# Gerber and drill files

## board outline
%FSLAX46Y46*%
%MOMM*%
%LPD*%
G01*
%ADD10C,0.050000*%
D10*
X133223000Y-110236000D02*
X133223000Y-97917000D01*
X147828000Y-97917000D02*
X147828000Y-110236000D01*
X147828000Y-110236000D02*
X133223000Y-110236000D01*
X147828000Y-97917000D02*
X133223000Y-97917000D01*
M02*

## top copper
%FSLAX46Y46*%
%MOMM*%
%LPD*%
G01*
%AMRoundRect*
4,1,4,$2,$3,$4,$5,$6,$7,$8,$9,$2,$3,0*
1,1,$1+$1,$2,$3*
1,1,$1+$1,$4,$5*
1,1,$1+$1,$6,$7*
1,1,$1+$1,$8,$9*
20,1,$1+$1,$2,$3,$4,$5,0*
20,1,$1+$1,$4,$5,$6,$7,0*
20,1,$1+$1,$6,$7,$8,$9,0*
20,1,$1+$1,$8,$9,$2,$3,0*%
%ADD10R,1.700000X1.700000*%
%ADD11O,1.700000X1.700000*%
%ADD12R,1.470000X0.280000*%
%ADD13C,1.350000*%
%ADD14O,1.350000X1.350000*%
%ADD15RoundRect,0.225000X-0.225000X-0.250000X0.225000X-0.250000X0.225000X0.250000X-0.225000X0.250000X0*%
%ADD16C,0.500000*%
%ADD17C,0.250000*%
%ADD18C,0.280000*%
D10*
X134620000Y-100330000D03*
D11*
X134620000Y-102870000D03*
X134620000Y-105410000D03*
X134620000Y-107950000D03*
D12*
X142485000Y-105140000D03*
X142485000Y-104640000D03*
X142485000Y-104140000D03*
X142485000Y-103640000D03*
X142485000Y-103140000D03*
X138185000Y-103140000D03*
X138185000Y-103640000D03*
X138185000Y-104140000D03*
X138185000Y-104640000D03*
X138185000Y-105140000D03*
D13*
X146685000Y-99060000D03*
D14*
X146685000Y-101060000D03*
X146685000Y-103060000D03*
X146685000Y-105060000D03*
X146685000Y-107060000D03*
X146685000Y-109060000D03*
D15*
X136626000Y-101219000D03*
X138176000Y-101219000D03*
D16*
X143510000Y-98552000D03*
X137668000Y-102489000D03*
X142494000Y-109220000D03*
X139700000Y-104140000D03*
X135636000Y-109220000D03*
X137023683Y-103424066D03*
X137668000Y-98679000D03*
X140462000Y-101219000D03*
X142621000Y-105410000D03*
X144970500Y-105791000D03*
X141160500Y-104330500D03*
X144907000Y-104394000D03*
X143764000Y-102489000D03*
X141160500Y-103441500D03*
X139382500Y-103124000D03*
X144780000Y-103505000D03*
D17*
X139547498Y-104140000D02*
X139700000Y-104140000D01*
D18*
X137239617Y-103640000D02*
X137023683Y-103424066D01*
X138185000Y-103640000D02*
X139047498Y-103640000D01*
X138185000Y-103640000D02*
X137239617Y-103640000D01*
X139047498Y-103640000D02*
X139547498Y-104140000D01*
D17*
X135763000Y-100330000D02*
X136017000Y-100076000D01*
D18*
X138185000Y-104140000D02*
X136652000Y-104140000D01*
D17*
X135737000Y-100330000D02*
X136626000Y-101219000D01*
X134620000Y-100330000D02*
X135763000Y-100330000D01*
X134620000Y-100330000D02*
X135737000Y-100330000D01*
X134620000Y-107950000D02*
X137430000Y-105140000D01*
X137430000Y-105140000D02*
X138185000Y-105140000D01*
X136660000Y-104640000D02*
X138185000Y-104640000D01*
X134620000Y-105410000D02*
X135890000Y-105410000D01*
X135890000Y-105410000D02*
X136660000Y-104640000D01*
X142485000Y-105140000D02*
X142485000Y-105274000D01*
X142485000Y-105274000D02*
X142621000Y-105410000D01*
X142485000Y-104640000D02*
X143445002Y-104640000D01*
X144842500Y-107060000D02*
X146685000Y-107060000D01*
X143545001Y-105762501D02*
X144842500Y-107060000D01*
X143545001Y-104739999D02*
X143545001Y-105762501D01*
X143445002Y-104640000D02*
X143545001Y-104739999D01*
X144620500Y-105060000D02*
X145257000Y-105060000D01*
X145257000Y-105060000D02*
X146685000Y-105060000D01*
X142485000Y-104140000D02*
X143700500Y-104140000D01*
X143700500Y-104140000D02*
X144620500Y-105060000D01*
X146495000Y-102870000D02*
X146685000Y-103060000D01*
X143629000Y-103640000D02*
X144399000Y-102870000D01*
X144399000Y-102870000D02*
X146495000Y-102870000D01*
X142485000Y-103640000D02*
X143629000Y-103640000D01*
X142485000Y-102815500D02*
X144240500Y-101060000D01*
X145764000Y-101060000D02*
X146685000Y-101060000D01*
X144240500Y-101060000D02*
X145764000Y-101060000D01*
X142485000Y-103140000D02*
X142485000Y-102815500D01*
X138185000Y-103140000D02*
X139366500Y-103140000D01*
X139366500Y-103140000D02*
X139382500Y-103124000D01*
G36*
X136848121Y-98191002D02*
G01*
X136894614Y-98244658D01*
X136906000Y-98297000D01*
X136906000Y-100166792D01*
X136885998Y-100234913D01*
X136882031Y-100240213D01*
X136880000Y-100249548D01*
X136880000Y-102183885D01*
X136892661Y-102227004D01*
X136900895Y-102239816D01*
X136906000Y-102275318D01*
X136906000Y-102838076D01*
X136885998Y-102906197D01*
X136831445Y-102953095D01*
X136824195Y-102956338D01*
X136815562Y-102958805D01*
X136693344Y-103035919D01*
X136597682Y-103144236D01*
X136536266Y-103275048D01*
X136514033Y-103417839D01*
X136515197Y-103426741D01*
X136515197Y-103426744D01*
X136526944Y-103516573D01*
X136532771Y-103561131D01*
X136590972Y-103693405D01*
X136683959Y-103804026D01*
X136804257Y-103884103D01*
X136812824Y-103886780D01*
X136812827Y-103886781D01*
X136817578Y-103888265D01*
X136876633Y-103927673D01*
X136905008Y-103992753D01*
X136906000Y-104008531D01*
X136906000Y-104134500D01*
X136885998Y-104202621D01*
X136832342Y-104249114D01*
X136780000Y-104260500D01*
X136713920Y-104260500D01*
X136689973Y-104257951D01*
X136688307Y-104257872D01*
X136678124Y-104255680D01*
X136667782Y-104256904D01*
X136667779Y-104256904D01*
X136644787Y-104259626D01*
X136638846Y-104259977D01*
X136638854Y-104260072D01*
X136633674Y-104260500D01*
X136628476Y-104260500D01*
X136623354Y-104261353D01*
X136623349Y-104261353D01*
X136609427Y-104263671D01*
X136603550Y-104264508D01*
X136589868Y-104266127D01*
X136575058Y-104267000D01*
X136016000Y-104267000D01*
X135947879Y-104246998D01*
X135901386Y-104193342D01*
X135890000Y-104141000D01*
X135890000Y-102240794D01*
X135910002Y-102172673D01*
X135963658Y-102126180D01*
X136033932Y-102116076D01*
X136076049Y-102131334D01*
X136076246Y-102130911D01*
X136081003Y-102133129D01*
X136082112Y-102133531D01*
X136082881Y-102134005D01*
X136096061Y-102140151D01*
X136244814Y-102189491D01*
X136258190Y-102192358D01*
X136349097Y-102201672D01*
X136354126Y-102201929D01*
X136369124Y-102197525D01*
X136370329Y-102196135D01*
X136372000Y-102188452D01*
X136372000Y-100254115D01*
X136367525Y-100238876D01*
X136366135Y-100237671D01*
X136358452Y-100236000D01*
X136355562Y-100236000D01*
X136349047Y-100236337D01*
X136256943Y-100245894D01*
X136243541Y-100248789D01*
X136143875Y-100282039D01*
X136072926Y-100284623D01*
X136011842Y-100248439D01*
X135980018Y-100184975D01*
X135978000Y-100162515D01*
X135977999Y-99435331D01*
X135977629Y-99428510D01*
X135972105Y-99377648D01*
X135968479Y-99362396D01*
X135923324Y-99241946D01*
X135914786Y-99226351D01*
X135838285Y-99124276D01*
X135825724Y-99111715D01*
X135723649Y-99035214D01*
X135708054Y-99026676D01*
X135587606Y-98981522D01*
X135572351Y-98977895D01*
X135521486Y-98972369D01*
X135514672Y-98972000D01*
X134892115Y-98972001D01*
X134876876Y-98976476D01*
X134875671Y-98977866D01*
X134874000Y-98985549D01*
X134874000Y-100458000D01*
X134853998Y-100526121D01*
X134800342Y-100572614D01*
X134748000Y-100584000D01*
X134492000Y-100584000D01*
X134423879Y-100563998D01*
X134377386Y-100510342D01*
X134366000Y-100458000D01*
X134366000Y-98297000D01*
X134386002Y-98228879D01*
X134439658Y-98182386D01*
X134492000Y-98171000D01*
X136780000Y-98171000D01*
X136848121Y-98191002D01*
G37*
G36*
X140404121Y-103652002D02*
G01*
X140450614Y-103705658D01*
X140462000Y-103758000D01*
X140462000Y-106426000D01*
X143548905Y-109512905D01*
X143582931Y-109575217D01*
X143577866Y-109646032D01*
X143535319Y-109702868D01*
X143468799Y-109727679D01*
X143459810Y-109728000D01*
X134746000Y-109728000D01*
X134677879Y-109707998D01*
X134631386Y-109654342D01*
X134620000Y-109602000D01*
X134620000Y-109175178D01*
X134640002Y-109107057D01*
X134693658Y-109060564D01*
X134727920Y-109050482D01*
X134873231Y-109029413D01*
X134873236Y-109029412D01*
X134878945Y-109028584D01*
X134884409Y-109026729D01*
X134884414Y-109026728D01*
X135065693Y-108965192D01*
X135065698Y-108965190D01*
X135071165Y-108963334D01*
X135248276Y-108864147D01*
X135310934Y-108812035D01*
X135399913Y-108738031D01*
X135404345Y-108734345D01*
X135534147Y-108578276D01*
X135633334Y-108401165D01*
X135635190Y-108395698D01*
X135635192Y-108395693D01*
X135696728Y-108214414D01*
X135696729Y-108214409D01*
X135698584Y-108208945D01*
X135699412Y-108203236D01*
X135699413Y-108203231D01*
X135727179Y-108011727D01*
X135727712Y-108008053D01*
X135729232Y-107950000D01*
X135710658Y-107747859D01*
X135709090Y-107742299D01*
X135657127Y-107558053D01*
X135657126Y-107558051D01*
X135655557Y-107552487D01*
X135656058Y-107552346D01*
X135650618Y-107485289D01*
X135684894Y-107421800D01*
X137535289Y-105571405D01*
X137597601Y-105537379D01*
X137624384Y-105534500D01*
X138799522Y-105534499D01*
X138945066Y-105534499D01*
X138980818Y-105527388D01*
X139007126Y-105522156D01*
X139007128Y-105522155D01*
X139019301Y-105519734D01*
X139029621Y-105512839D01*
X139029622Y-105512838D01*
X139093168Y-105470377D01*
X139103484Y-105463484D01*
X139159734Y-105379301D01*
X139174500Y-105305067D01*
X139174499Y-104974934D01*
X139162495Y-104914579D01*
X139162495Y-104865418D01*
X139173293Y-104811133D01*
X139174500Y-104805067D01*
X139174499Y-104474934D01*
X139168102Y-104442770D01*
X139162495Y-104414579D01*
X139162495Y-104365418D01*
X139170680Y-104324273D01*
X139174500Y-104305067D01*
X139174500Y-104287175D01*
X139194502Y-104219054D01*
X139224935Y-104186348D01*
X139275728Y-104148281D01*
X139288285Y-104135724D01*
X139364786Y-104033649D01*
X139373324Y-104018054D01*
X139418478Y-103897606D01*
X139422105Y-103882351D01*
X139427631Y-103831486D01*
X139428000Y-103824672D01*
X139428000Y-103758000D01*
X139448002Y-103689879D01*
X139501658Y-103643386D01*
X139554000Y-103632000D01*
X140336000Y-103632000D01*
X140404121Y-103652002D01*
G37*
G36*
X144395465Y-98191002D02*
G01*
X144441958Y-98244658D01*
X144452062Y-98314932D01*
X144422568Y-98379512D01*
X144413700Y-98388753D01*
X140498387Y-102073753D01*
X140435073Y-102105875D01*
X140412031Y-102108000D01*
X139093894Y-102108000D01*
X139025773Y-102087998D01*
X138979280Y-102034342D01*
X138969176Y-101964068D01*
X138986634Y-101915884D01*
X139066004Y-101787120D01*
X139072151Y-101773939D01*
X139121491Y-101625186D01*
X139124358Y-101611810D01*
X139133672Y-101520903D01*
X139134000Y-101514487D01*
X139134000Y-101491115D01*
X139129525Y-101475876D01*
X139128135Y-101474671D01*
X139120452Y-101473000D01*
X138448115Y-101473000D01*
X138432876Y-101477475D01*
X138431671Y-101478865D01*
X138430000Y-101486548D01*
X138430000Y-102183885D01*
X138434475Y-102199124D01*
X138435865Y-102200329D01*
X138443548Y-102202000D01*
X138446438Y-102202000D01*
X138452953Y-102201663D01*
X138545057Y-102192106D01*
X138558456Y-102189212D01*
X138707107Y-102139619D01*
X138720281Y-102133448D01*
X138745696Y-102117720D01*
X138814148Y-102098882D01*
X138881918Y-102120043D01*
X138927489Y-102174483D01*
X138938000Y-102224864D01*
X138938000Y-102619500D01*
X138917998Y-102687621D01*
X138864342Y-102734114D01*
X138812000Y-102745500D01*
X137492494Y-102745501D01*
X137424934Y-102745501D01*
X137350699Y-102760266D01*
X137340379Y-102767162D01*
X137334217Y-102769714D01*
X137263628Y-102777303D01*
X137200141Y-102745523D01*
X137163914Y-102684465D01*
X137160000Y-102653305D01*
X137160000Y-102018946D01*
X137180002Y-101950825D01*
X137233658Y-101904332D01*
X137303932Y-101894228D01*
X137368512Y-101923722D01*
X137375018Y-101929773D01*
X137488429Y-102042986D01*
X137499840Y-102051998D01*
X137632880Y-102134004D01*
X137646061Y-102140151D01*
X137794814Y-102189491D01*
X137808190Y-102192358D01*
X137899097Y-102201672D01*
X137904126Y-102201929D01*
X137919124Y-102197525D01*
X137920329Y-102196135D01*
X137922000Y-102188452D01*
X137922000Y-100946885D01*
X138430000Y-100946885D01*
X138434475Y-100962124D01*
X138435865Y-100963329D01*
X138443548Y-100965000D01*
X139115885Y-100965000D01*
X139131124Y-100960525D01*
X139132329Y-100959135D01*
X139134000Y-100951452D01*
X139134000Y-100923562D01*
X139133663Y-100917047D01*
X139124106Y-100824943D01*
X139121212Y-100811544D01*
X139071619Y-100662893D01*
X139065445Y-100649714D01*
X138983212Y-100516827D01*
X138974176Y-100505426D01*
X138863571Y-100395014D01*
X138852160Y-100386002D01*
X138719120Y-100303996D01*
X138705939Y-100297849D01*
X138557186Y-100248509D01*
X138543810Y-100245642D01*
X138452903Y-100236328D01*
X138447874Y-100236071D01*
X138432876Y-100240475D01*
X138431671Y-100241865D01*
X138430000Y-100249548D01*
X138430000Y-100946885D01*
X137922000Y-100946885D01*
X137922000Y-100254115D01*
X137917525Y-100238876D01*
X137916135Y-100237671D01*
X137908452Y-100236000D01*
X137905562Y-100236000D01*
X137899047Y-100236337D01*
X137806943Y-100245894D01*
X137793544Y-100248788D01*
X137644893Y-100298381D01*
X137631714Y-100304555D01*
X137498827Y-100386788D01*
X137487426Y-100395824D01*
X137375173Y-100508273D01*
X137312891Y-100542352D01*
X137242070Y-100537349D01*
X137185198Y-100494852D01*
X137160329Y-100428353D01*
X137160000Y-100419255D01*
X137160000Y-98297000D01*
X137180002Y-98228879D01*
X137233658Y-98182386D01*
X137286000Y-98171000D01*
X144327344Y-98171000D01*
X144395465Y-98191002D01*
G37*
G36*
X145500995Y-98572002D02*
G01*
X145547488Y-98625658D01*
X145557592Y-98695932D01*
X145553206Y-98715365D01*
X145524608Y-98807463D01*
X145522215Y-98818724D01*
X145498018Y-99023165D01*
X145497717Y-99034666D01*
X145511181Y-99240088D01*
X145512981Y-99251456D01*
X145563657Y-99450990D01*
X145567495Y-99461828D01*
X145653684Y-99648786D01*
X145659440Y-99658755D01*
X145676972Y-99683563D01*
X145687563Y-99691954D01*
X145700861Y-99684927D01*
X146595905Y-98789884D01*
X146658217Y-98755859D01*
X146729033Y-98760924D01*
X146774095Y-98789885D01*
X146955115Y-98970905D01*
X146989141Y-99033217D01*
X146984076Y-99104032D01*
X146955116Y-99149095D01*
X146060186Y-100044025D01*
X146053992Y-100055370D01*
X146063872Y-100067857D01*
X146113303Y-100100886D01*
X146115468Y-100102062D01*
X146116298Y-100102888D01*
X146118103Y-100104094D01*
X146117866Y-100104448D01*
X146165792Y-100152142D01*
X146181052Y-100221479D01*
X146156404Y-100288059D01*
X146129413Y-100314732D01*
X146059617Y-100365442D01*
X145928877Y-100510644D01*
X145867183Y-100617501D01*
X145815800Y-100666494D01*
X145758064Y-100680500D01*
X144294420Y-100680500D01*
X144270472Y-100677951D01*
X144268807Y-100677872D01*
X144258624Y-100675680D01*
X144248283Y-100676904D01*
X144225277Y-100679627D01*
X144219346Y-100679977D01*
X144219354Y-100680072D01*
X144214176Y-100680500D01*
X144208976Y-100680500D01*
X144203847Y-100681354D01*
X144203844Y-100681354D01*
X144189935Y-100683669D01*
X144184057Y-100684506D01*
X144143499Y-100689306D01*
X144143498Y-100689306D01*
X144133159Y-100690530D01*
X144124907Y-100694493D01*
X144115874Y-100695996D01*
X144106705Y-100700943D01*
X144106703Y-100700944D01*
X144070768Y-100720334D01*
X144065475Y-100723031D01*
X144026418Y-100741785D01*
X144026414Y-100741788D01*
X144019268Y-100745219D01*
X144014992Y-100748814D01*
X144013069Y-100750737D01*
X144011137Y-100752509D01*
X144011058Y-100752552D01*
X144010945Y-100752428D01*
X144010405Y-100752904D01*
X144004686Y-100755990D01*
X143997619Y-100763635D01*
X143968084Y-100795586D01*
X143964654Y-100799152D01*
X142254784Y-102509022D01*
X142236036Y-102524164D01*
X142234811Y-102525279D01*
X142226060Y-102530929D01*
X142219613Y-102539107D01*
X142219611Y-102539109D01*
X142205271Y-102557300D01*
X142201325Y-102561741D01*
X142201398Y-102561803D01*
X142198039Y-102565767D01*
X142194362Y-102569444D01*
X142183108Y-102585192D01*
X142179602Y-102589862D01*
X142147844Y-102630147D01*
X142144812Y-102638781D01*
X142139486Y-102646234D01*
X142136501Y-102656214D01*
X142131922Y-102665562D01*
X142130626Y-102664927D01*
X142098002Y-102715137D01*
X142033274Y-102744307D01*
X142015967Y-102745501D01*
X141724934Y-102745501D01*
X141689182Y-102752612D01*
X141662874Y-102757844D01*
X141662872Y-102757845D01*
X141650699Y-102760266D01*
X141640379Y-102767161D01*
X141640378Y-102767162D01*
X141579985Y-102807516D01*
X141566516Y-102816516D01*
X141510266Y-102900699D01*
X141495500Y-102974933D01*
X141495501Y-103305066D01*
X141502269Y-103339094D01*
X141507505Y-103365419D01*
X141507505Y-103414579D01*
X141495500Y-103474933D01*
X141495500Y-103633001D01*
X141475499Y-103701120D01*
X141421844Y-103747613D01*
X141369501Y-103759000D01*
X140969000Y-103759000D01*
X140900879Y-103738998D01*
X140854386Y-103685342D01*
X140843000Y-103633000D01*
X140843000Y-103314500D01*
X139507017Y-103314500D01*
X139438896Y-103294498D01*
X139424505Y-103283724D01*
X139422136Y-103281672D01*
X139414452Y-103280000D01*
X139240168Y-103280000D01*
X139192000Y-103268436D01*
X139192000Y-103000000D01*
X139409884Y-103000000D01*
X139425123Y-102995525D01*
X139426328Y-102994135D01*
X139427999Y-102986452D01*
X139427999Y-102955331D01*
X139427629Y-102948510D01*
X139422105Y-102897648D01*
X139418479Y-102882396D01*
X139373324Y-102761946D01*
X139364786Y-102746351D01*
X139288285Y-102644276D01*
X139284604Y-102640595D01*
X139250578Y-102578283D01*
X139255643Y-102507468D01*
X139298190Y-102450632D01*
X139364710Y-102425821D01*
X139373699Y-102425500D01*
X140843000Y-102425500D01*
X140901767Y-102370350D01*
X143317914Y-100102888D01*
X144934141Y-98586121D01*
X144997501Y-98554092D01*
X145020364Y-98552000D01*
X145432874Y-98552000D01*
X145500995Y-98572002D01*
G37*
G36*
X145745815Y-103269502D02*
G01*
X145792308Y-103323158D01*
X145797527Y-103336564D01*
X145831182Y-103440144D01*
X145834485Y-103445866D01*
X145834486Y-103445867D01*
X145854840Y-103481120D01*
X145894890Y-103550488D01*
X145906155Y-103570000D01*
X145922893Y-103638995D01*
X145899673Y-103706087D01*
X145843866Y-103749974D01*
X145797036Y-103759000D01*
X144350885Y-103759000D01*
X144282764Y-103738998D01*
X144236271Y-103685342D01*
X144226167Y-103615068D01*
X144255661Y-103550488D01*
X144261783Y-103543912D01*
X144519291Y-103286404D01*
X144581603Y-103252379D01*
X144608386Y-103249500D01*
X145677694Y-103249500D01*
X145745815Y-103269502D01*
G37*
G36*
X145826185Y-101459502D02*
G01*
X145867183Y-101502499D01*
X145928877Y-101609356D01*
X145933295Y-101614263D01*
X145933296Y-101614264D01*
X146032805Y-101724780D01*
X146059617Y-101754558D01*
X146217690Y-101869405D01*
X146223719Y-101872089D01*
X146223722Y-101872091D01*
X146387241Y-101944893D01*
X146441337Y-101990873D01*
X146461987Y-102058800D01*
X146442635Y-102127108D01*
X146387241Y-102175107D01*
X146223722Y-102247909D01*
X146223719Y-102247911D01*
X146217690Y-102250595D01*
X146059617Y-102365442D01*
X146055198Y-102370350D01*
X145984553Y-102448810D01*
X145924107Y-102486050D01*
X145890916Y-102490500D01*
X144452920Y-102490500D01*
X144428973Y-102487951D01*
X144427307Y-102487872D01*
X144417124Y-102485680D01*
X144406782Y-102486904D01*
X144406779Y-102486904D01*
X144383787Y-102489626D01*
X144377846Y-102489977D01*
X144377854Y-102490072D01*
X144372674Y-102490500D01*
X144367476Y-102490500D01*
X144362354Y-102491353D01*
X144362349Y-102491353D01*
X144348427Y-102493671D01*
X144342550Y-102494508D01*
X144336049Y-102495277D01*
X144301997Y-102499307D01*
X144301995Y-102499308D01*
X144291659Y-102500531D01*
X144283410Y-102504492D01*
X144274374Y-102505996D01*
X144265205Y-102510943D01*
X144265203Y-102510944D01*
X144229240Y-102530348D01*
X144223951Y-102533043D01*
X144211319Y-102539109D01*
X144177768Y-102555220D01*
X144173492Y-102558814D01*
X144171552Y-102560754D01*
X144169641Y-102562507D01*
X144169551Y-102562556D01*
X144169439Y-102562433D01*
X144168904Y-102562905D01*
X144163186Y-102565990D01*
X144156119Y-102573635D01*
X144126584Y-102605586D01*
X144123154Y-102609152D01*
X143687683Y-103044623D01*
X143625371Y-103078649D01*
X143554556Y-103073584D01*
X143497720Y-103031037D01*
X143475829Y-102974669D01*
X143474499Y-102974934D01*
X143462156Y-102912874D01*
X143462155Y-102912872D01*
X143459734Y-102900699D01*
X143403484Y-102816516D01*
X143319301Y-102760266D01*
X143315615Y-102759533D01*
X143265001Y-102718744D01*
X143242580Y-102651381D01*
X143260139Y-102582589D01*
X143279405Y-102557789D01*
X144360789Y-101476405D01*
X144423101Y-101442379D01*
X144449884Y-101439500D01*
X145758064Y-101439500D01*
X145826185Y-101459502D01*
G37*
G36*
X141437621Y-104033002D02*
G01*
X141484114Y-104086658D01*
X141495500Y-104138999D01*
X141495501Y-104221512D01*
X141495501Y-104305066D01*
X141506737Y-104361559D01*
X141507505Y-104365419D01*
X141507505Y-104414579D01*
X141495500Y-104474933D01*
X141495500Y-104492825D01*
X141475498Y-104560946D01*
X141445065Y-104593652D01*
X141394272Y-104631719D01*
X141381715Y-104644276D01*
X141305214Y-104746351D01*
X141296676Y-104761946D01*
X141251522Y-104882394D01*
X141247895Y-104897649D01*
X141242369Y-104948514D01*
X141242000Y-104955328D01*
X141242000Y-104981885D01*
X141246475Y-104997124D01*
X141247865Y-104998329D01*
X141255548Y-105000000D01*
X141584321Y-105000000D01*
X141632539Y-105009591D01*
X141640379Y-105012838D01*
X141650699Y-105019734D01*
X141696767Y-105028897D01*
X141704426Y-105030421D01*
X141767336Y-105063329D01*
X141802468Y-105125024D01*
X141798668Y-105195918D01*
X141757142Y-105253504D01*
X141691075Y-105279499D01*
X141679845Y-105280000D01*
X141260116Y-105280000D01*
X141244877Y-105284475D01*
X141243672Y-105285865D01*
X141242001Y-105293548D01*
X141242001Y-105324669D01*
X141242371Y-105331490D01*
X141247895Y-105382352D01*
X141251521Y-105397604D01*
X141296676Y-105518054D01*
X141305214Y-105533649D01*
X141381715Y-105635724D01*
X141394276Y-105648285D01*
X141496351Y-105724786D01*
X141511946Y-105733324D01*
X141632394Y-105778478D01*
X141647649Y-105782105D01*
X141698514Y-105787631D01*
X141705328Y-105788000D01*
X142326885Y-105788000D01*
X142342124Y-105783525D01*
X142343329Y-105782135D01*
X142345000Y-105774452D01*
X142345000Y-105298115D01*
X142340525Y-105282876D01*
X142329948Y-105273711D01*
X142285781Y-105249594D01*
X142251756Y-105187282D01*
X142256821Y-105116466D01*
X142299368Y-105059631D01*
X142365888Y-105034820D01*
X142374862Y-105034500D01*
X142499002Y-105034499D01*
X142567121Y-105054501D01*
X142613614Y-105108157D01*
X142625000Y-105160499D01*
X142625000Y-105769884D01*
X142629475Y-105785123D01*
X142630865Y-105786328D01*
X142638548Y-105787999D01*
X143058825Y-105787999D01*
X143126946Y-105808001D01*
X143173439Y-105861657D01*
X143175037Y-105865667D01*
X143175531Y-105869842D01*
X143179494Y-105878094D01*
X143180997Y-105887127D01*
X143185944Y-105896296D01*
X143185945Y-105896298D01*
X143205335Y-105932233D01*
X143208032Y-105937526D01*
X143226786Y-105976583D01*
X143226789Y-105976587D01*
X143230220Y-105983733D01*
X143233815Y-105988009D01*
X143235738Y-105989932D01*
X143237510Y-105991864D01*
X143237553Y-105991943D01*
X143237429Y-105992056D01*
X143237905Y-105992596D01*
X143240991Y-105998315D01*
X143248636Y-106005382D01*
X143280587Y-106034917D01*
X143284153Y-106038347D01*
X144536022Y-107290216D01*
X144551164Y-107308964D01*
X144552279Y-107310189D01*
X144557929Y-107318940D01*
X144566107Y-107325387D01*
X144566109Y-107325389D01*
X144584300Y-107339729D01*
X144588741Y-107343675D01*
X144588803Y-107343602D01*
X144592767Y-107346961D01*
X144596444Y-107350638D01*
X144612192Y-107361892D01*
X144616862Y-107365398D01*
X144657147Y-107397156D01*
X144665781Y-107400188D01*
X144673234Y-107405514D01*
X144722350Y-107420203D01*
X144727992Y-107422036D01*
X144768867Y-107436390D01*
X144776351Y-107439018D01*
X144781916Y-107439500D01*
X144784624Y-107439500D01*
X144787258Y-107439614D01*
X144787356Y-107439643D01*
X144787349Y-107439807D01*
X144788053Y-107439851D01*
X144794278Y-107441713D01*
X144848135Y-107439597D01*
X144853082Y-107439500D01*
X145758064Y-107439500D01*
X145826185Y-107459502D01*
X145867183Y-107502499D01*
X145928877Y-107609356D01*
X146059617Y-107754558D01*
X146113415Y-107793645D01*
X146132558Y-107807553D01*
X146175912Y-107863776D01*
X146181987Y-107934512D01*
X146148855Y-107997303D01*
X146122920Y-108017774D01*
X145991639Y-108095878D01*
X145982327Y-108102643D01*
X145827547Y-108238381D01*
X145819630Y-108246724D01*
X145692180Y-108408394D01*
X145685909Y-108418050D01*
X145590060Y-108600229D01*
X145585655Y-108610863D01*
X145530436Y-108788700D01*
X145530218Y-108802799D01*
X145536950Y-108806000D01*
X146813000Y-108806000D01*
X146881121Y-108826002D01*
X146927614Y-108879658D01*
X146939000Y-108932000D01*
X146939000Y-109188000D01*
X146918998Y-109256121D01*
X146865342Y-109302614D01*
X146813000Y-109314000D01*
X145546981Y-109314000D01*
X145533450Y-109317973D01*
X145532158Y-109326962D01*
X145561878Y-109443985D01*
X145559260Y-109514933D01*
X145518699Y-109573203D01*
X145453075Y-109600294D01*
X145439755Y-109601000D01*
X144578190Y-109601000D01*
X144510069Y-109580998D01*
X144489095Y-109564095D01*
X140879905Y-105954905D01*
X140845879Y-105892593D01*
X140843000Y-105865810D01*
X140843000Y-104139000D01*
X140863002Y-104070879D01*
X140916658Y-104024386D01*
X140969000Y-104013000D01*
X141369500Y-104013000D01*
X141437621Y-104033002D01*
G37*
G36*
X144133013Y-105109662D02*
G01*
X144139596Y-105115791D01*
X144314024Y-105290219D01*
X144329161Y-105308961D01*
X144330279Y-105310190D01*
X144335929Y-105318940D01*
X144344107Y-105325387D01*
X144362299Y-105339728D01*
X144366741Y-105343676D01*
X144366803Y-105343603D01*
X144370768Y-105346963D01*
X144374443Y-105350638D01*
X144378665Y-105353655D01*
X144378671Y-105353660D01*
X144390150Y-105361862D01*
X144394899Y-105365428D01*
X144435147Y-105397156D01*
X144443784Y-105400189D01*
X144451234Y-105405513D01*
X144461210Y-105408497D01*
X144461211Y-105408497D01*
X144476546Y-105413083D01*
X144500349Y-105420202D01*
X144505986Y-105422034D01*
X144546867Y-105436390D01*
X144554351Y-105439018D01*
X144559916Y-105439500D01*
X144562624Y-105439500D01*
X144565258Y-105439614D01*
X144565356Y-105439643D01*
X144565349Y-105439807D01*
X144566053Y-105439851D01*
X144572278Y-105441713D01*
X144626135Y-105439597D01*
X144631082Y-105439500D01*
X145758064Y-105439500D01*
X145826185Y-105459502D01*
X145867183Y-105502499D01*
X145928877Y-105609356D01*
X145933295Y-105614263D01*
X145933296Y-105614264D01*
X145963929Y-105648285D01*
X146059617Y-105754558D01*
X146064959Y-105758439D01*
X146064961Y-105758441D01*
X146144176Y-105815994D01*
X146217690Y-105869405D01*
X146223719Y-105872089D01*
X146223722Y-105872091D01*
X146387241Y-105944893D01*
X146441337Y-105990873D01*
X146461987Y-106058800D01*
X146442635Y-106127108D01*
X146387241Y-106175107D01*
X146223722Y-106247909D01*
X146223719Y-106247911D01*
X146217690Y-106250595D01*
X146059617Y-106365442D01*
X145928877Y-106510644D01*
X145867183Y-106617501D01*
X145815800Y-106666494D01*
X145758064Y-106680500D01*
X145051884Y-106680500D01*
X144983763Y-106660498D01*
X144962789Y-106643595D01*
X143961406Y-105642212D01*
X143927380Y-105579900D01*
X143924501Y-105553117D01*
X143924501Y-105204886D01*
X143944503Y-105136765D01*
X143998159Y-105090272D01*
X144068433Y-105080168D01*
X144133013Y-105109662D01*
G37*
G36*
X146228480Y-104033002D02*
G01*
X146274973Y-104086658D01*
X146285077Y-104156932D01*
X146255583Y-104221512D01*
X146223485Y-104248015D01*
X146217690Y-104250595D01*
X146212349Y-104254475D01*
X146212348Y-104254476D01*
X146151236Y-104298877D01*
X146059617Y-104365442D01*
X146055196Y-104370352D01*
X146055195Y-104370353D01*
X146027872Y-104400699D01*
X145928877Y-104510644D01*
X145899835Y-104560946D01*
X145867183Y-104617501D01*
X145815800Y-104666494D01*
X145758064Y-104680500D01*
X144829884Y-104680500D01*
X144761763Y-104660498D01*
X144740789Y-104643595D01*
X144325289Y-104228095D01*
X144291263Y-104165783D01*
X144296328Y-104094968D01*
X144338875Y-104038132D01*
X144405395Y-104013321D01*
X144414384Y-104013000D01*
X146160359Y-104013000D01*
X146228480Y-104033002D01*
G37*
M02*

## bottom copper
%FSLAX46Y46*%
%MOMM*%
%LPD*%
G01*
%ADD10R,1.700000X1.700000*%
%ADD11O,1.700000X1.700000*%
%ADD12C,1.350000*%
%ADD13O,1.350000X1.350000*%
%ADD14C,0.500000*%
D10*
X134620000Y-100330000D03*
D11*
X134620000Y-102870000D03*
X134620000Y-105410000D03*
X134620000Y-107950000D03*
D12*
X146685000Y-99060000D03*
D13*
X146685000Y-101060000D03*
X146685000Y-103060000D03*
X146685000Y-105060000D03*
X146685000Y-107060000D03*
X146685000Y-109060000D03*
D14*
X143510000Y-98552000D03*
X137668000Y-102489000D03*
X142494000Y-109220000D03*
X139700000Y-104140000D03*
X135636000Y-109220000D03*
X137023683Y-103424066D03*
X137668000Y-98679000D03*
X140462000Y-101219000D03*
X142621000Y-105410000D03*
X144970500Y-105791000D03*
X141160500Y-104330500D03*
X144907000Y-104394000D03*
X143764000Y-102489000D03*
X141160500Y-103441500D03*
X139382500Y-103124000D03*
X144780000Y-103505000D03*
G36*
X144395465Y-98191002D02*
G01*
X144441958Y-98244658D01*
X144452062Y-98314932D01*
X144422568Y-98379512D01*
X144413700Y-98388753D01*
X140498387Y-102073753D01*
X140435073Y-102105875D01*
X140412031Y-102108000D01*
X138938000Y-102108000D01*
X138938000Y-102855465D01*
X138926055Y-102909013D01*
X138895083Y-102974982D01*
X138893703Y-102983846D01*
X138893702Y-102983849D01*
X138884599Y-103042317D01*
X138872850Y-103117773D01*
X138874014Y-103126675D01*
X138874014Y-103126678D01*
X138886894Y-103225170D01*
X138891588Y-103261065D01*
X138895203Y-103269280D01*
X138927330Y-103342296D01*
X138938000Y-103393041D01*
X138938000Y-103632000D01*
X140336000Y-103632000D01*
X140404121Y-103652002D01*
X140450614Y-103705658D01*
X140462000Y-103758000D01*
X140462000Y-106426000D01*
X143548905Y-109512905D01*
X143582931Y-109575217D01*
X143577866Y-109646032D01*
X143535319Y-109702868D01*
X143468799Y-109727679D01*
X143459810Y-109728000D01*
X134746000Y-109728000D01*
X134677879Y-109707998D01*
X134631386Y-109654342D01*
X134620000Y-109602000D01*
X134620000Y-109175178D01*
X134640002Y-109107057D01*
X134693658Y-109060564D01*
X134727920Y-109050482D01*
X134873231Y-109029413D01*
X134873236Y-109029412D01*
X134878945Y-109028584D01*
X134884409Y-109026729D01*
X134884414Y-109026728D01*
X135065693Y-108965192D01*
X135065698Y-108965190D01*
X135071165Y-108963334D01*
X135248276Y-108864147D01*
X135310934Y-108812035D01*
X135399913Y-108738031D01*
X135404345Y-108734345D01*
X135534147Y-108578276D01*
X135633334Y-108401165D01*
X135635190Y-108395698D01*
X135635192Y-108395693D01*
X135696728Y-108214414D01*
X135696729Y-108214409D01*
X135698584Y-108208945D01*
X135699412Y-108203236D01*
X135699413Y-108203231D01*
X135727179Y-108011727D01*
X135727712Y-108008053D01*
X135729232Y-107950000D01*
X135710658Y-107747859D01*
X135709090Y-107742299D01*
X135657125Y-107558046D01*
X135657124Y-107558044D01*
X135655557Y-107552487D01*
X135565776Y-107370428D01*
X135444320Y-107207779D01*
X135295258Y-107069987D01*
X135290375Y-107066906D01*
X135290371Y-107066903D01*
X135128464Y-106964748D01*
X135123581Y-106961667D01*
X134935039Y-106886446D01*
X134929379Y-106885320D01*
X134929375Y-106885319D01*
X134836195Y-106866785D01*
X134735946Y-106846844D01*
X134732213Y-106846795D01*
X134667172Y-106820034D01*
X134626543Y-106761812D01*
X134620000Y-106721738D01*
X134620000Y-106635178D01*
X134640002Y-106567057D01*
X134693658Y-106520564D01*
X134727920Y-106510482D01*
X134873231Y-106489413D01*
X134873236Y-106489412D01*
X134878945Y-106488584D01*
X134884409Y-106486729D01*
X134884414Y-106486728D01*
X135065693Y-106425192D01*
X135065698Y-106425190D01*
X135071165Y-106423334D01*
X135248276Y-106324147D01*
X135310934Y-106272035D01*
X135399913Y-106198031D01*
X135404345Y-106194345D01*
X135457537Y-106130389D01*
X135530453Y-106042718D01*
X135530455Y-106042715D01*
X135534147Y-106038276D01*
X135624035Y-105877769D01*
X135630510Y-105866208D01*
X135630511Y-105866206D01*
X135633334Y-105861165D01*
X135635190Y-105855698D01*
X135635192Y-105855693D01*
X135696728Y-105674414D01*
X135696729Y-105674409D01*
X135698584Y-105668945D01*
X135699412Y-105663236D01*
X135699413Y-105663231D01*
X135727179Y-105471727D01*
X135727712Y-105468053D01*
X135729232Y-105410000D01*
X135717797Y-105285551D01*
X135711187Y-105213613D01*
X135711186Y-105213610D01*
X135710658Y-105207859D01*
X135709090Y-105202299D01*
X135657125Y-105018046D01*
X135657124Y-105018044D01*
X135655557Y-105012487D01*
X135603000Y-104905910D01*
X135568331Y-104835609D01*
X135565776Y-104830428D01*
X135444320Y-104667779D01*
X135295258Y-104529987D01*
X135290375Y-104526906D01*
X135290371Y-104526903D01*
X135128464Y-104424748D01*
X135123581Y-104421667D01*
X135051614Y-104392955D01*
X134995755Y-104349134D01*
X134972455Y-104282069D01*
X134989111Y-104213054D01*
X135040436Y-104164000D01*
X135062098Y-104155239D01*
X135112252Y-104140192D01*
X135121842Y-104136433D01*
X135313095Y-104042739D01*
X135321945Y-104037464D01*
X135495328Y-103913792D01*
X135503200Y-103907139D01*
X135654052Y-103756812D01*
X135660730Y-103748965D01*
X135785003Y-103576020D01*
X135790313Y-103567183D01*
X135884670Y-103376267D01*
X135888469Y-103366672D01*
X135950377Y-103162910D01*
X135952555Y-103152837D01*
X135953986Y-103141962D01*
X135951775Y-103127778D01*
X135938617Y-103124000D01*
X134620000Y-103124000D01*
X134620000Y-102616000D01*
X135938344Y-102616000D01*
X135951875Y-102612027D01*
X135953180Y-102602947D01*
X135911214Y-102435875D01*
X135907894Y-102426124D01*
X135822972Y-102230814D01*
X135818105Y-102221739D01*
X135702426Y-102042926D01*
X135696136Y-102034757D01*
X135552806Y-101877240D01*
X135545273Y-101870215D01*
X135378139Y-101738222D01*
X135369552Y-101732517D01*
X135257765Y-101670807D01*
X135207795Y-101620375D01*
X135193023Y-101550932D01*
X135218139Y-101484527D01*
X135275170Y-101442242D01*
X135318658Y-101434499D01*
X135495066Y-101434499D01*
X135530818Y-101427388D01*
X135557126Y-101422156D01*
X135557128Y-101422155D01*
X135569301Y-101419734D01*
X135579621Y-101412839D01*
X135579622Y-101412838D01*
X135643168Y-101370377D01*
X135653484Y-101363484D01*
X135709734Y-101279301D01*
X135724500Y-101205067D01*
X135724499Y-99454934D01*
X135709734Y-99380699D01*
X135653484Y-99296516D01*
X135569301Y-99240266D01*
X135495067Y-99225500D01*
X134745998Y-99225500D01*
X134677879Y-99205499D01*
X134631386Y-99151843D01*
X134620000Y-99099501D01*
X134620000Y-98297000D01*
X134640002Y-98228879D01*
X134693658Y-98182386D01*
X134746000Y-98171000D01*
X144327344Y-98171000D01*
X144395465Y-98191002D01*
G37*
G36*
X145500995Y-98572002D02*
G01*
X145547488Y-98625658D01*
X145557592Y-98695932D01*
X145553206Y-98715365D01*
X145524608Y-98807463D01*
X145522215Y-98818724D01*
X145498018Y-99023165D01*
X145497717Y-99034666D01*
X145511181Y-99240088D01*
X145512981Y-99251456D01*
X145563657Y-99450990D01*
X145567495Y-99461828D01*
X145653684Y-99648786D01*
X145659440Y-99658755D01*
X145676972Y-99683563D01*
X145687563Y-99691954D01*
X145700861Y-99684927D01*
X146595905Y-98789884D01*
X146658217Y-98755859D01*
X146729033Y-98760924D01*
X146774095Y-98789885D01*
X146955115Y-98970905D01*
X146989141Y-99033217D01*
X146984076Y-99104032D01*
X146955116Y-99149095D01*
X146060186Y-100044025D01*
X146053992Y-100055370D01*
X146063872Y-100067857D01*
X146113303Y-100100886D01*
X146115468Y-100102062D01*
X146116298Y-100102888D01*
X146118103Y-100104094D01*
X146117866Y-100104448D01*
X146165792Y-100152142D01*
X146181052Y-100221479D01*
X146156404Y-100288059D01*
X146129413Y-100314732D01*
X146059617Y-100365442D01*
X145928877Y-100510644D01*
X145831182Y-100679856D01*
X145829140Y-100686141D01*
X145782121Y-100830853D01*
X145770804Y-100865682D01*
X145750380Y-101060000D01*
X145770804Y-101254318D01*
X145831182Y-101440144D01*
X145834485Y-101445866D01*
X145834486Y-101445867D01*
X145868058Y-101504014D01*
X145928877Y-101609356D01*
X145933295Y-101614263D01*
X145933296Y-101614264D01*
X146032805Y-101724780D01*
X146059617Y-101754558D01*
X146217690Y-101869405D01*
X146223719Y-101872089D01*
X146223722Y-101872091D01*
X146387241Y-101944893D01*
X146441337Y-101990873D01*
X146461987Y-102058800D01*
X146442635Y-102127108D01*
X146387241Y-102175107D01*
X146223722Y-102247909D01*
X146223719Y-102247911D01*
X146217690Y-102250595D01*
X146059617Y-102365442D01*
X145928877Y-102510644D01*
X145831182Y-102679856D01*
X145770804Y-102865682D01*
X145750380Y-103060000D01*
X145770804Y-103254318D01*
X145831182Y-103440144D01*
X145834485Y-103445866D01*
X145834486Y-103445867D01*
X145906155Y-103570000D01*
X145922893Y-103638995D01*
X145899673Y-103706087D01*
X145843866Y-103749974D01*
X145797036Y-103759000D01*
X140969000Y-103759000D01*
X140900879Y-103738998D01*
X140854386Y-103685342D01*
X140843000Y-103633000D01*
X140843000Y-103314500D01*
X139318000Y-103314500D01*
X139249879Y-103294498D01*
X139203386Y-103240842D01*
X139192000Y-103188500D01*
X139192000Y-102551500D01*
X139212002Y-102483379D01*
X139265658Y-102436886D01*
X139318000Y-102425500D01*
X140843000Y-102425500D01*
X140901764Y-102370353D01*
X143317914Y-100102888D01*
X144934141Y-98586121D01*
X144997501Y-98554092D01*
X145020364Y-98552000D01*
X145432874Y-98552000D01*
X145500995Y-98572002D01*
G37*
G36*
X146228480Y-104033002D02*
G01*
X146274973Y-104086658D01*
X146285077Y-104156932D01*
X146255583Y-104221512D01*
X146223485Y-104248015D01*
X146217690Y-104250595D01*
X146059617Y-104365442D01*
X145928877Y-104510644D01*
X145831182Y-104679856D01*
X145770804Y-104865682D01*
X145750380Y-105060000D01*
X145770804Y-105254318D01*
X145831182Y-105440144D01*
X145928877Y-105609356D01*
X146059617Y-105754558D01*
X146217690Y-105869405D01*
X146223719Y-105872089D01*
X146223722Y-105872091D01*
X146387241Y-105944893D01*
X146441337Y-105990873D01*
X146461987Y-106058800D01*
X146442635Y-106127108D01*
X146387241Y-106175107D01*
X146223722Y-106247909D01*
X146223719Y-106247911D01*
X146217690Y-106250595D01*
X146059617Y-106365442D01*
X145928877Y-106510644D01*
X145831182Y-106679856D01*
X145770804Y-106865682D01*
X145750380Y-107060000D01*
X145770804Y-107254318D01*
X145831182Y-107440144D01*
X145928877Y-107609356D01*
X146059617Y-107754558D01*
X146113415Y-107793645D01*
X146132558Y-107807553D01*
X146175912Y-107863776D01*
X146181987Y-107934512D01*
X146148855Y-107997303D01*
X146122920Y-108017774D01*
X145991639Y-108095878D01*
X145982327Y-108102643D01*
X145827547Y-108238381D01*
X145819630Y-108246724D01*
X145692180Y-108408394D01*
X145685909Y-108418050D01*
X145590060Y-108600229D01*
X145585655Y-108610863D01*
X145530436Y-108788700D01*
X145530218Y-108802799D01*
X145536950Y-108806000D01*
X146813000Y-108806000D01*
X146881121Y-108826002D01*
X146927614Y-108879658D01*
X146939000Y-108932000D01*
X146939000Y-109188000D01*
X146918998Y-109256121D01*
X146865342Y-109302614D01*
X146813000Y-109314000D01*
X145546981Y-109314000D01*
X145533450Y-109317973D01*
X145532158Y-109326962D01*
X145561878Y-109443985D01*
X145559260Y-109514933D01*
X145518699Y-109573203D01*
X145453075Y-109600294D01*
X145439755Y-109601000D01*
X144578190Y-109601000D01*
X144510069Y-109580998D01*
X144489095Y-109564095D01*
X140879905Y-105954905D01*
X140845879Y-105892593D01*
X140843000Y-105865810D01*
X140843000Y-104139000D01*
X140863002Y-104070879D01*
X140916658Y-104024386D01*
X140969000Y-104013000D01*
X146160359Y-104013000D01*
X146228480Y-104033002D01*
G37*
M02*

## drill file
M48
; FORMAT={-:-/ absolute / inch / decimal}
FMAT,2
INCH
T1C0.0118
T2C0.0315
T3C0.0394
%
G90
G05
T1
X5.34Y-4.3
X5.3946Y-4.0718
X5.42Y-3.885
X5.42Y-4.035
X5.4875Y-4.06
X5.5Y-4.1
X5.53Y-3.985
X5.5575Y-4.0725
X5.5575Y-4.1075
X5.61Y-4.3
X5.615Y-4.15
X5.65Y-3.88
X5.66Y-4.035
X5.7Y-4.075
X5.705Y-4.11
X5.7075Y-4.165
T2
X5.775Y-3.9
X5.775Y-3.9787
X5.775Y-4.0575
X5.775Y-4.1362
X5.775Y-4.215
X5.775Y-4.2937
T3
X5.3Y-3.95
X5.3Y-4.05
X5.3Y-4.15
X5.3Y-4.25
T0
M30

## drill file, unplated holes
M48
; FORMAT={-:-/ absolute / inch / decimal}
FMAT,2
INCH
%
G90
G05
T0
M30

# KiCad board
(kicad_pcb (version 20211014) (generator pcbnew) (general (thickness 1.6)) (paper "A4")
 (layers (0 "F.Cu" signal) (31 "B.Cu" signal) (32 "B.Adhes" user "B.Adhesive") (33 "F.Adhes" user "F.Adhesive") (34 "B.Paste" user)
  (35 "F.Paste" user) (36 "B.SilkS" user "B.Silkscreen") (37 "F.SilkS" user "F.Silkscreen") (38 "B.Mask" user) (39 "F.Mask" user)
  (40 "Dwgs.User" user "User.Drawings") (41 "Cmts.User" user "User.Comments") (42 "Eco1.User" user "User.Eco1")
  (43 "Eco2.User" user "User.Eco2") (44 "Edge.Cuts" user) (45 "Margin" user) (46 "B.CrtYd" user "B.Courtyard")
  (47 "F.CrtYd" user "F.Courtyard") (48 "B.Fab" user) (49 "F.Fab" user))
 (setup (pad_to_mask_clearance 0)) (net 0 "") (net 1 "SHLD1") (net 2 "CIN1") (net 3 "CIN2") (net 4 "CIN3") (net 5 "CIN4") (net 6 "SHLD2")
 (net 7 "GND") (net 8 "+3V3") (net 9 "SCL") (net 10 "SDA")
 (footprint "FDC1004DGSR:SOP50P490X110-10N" (layer "F.Cu") (at 140.335 104.14 180)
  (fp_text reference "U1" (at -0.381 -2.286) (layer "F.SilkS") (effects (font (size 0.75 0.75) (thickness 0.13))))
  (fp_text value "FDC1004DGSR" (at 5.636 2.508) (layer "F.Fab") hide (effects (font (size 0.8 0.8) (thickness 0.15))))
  (pad "1" smd rect locked (at -2.15 -1 180) (size 1.47 0.28) (layers "F.Cu" "F.Paste" "F.Mask") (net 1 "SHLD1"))
  (pad "2" smd rect locked (at -2.15 -0.5 180) (size 1.47 0.28) (layers "F.Cu" "F.Paste" "F.Mask") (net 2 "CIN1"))
  (pad "3" smd rect locked (at -2.15 0 180) (size 1.47 0.28) (layers "F.Cu" "F.Paste" "F.Mask") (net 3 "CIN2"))
  (pad "4" smd rect locked (at -2.15 0.5 180) (size 1.47 0.28) (layers "F.Cu" "F.Paste" "F.Mask") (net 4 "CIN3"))
  (pad "5" smd rect locked (at -2.15 1 180) (size 1.47 0.28) (layers "F.Cu" "F.Paste" "F.Mask") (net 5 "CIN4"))
  (pad "6" smd rect locked (at 2.15 1 180) (size 1.47 0.28) (layers "F.Cu" "F.Paste" "F.Mask") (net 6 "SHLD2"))
  (pad "7" smd rect locked (at 2.15 0.5 180) (size 1.47 0.28) (layers "F.Cu" "F.Paste" "F.Mask") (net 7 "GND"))
  (pad "8" smd rect locked (at 2.15 0 180) (size 1.47 0.28) (layers "F.Cu" "F.Paste" "F.Mask") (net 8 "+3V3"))
  (pad "9" smd rect locked (at 2.15 -0.5 180) (size 1.47 0.28) (layers "F.Cu" "F.Paste" "F.Mask") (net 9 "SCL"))
  (pad "10" smd rect locked (at 2.15 -1 180) (size 1.47 0.28) (layers "F.Cu" "F.Paste" "F.Mask") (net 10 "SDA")))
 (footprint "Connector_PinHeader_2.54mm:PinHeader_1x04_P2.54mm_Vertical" (layer "F.Cu") (at 134.62 100.33)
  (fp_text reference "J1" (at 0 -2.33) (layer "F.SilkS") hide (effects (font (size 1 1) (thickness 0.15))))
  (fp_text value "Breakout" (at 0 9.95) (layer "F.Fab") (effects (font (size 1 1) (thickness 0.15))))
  (pad "1" thru_hole rect (at 0 0) (size 1.7 1.7) (drill 1) (layers *.Cu *.Mask) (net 8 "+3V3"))
  (pad "2" thru_hole oval (at 0 2.54) (size 1.7 1.7) (drill 1) (layers *.Cu *.Mask) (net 7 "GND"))
  (pad "3" thru_hole oval (at 0 5.08) (size 1.7 1.7) (drill 1) (layers *.Cu *.Mask) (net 9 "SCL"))
  (pad "4" thru_hole oval (at 0 7.62) (size 1.7 1.7) (drill 1) (layers *.Cu *.Mask) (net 10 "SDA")))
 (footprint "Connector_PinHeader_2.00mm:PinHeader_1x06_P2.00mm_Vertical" (layer "F.Cu") (at 146.685 99.06)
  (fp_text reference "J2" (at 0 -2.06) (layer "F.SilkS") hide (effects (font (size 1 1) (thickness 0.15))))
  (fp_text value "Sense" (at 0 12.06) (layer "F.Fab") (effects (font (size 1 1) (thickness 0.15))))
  (pad "1" thru_hole circle locked (at 0 0) (size 1.35 1.35) (drill 0.8) (layers *.Cu *.Mask) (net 6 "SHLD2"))
  (pad "2" thru_hole oval locked (at 0 2) (size 1.35 1.35) (drill 0.8) (layers *.Cu *.Mask) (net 5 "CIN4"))
  (pad "3" thru_hole oval locked (at 0 4) (size 1.35 1.35) (drill 0.8) (layers *.Cu *.Mask) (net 4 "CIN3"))
  (pad "4" thru_hole oval locked (at 0 6) (size 1.35 1.35) (drill 0.8) (layers *.Cu *.Mask) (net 3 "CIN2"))
  (pad "5" thru_hole oval locked (at 0 8) (size 1.35 1.35) (drill 0.8) (layers *.Cu *.Mask) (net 2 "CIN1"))
  (pad "6" thru_hole oval locked (at 0 10) (size 1.35 1.35) (drill 0.8) (layers *.Cu *.Mask) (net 1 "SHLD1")))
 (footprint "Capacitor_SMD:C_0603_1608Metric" (layer "F.Cu") (at 137.401 101.219)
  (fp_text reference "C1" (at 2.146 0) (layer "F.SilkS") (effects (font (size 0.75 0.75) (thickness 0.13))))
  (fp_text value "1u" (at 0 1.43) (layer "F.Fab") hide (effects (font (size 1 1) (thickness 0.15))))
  (pad "1" smd roundrect locked (at -0.775 0) (size 0.9 0.95) (layers "F.Cu" "F.Paste" "F.Mask") (roundrect_rratio 0.25) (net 8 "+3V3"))
  (pad "2" smd roundrect locked (at 0.775 0) (size 0.9 0.95) (layers "F.Cu" "F.Paste" "F.Mask") (roundrect_rratio 0.25) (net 7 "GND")))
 (gr_line (start 133.223 110.236) (end 133.223 97.917) (layer "Edge.Cuts") (width 0.05))
 (gr_line (start 147.828 97.917) (end 147.828 110.236) (layer "Edge.Cuts") (width 0.05))
 (gr_line (start 147.828 110.236) (end 133.223 110.236) (layer "Edge.Cuts") (width 0.05))
 (gr_line (start 147.828 97.917) (end 133.223 97.917) (layer "Edge.Cuts") (width 0.05))
 (segment (start 139.547498 104.14) (end 139.7 104.14) (width 0.25) (layer "F.Cu") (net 7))
 (segment (start 137.239617 103.64) (end 137.023683 103.424066) (width 0.28) (layer "F.Cu") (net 7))
 (segment (start 138.185 103.64) (end 139.047498 103.64) (width 0.28) (layer "F.Cu") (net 7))
 (segment (start 138.185 103.64) (end 137.239617 103.64) (width 0.28) (layer "F.Cu") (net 7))
 (segment (start 139.047498 103.64) (end 139.547498 104.14) (width 0.28) (layer "F.Cu") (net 7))
 (via (at 143.51 98.552) (size 0.5) (drill 0.3) (layers "F.Cu" "B.Cu") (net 7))
 (via (at 137.668 102.489) (size 0.5) (drill 0.3) (layers "F.Cu" "B.Cu") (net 7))
 (via (at 142.494 109.22) (size 0.5) (drill 0.3) (layers "F.Cu" "B.Cu") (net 7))
 (via (at 139.7 104.14) (size 0.5) (drill 0.3) (layers "F.Cu" "B.Cu") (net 7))
 (via (at 135.636 109.22) (size 0.5) (drill 0.3) (layers "F.Cu" "B.Cu") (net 7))
 (via (at 137.023683 103.424066) (size 0.5) (drill 0.3) (layers "F.Cu" "B.Cu") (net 7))
 (via (at 137.668 98.679) (size 0.5) (drill 0.3) (layers "F.Cu" "B.Cu") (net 7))
 (via (at 140.462 101.219) (size 0.5) (drill 0.3) (layers "F.Cu" "B.Cu") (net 7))
 (segment (start 135.763 100.33) (end 136.017 100.076) (width 0.25) (layer "F.Cu") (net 8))
 (segment (start 138.185 104.14) (end 136.652 104.14) (width 0.28) (layer "F.Cu") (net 8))
 (segment (start 135.737 100.33) (end 136.626 101.219) (width 0.25) (layer "F.Cu") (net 8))
 (segment (start 134.62 100.33) (end 135.763 100.33) (width 0.25) (layer "F.Cu") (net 8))
 (segment (start 134.62 100.33) (end 135.737 100.33) (width 0.25) (layer "F.Cu") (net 8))
 (segment (start 134.62 107.95) (end 137.43 105.14) (width 0.25) (layer "F.Cu") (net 10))
 (segment (start 137.43 105.14) (end 138.185 105.14) (width 0.25) (layer "F.Cu") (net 10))
 (segment (start 136.66 104.64) (end 138.185 104.64) (width 0.25) (layer "F.Cu") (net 9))
 (segment (start 134.62 105.41) (end 135.89 105.41) (width 0.25) (layer "F.Cu") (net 9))
 (segment (start 135.89 105.41) (end 136.66 104.64) (width 0.25) (layer "F.Cu") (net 9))
 (segment (start 142.485 105.14) (end 142.485 105.274) (width 0.25) (layer "F.Cu") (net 1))
 (segment (start 142.485 105.274) (end 142.621 105.41) (width 0.25) (layer "F.Cu") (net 1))
 (via (at 142.621 105.41) (size 0.5) (drill 0.3) (layers "F.Cu" "B.Cu") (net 1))
 (via (at 144.9705 105.791) (size 0.5) (drill 0.3) (layers "F.Cu" "B.Cu") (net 1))
 (via (at 141.1605 104.3305) (size 0.5) (drill 0.3) (layers "F.Cu" "B.Cu") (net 1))
 (via (at 144.907 104.394) (size 0.5) (drill 0.3) (layers "F.Cu" "B.Cu") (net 1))
 (segment (start 142.485 104.64) (end 143.445002 104.64) (width 0.25) (layer "F.Cu") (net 2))
 (segment (start 144.8425 107.06) (end 146.685 107.06) (width 0.25) (layer "F.Cu") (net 2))
 (segment (start 143.545001 105.762501) (end 144.8425 107.06) (width 0.25) (layer "F.Cu") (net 2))
 (segment (start 143.545001 104.739999) (end 143.545001 105.762501) (width 0.25) (layer "F.Cu") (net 2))
 (segment (start 143.445002 104.64) (end 143.545001 104.739999) (width 0.25) (layer "F.Cu") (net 2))
 (segment (start 144.6205 105.06) (end 145.257 105.06) (width 0.25) (layer "F.Cu") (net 3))
 (segment (start 145.257 105.06) (end 146.685 105.06) (width 0.25) (layer "F.Cu") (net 3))
 (segment (start 142.485 104.14) (end 143.7005 104.14) (width 0.25) (layer "F.Cu") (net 3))
 (segment (start 143.7005 104.14) (end 144.6205 105.06) (width 0.25) (layer "F.Cu") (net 3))
 (segment (start 146.495 102.87) (end 146.685 103.06) (width 0.25) (layer "F.Cu") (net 4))
 (segment (start 143.629 103.64) (end 144.399 102.87) (width 0.25) (layer "F.Cu") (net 4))
 (segment (start 144.399 102.87) (end 146.495 102.87) (width 0.25) (layer "F.Cu") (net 4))
 (segment (start 142.485 103.64) (end 143.629 103.64) (width 0.25) (layer "F.Cu") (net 4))
 (segment (start 142.485 102.8155) (end 144.2405 101.06) (width 0.25) (layer "F.Cu") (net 5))
 (segment (start 145.764 101.06) (end 146.685 101.06) (width 0.25) (layer "F.Cu") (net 5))
 (segment (start 144.2405 101.06) (end 145.764 101.06) (width 0.25) (layer "F.Cu") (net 5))
 (segment (start 142.485 103.14) (end 142.485 102.8155) (width 0.25) (layer "F.Cu") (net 5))
 (segment (start 138.185 103.14) (end 139.3665 103.14) (width 0.25) (layer "F.Cu") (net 6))
 (segment (start 139.3665 103.14) (end 139.3825 103.124) (width 0.25) (layer "F.Cu") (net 6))
 (via (at 143.764 102.489) (size 0.5) (drill 0.3) (layers "F.Cu" "B.Cu") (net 6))
 (via (at 141.1605 103.4415) (size 0.5) (drill 0.3) (layers "F.Cu" "B.Cu") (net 6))
 (via (at 139.3825 103.124) (size 0.5) (drill 0.3) (layers "F.Cu" "B.Cu") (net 6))
 (via (at 144.78 103.505) (size 0.5) (drill 0.3) (layers "F.Cu" "B.Cu") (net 6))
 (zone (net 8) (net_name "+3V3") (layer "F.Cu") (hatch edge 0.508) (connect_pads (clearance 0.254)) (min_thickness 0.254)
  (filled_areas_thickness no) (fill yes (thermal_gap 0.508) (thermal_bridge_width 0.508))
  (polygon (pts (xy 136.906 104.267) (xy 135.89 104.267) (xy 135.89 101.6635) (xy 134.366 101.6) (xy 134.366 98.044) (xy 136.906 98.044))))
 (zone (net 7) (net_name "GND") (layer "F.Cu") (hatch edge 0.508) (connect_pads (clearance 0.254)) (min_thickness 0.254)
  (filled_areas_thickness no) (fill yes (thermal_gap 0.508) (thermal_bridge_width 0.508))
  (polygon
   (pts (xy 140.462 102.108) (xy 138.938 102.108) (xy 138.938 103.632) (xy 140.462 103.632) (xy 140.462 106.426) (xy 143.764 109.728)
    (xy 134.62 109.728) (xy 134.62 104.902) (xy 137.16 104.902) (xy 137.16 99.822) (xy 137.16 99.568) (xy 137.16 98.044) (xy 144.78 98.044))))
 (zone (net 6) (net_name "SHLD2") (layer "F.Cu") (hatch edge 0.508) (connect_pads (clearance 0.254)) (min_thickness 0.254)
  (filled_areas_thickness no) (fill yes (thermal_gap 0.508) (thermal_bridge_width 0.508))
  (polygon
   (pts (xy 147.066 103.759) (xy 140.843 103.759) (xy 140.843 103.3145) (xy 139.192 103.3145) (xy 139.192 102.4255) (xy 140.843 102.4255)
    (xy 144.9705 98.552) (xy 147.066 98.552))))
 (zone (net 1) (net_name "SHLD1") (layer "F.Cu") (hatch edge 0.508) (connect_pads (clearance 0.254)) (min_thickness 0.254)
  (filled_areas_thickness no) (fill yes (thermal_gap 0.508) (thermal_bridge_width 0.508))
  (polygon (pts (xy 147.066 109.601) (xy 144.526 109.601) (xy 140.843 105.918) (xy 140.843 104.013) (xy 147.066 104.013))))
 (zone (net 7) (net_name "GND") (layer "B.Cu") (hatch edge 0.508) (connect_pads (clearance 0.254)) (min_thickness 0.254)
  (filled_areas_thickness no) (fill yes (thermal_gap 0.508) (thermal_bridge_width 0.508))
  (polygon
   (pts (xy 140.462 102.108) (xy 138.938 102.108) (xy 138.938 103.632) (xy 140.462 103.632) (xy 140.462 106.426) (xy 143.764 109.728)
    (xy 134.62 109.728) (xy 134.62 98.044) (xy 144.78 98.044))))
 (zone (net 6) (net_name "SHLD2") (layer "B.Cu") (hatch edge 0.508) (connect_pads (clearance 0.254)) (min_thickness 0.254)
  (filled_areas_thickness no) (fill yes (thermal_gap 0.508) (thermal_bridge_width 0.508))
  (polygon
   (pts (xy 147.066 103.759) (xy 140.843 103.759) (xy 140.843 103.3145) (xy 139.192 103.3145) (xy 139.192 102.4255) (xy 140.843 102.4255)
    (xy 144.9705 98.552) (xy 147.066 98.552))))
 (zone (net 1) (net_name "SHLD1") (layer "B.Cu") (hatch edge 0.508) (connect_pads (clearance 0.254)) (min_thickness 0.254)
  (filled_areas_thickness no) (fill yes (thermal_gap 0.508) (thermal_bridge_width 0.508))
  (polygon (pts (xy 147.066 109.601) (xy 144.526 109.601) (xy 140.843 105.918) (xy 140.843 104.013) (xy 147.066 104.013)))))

